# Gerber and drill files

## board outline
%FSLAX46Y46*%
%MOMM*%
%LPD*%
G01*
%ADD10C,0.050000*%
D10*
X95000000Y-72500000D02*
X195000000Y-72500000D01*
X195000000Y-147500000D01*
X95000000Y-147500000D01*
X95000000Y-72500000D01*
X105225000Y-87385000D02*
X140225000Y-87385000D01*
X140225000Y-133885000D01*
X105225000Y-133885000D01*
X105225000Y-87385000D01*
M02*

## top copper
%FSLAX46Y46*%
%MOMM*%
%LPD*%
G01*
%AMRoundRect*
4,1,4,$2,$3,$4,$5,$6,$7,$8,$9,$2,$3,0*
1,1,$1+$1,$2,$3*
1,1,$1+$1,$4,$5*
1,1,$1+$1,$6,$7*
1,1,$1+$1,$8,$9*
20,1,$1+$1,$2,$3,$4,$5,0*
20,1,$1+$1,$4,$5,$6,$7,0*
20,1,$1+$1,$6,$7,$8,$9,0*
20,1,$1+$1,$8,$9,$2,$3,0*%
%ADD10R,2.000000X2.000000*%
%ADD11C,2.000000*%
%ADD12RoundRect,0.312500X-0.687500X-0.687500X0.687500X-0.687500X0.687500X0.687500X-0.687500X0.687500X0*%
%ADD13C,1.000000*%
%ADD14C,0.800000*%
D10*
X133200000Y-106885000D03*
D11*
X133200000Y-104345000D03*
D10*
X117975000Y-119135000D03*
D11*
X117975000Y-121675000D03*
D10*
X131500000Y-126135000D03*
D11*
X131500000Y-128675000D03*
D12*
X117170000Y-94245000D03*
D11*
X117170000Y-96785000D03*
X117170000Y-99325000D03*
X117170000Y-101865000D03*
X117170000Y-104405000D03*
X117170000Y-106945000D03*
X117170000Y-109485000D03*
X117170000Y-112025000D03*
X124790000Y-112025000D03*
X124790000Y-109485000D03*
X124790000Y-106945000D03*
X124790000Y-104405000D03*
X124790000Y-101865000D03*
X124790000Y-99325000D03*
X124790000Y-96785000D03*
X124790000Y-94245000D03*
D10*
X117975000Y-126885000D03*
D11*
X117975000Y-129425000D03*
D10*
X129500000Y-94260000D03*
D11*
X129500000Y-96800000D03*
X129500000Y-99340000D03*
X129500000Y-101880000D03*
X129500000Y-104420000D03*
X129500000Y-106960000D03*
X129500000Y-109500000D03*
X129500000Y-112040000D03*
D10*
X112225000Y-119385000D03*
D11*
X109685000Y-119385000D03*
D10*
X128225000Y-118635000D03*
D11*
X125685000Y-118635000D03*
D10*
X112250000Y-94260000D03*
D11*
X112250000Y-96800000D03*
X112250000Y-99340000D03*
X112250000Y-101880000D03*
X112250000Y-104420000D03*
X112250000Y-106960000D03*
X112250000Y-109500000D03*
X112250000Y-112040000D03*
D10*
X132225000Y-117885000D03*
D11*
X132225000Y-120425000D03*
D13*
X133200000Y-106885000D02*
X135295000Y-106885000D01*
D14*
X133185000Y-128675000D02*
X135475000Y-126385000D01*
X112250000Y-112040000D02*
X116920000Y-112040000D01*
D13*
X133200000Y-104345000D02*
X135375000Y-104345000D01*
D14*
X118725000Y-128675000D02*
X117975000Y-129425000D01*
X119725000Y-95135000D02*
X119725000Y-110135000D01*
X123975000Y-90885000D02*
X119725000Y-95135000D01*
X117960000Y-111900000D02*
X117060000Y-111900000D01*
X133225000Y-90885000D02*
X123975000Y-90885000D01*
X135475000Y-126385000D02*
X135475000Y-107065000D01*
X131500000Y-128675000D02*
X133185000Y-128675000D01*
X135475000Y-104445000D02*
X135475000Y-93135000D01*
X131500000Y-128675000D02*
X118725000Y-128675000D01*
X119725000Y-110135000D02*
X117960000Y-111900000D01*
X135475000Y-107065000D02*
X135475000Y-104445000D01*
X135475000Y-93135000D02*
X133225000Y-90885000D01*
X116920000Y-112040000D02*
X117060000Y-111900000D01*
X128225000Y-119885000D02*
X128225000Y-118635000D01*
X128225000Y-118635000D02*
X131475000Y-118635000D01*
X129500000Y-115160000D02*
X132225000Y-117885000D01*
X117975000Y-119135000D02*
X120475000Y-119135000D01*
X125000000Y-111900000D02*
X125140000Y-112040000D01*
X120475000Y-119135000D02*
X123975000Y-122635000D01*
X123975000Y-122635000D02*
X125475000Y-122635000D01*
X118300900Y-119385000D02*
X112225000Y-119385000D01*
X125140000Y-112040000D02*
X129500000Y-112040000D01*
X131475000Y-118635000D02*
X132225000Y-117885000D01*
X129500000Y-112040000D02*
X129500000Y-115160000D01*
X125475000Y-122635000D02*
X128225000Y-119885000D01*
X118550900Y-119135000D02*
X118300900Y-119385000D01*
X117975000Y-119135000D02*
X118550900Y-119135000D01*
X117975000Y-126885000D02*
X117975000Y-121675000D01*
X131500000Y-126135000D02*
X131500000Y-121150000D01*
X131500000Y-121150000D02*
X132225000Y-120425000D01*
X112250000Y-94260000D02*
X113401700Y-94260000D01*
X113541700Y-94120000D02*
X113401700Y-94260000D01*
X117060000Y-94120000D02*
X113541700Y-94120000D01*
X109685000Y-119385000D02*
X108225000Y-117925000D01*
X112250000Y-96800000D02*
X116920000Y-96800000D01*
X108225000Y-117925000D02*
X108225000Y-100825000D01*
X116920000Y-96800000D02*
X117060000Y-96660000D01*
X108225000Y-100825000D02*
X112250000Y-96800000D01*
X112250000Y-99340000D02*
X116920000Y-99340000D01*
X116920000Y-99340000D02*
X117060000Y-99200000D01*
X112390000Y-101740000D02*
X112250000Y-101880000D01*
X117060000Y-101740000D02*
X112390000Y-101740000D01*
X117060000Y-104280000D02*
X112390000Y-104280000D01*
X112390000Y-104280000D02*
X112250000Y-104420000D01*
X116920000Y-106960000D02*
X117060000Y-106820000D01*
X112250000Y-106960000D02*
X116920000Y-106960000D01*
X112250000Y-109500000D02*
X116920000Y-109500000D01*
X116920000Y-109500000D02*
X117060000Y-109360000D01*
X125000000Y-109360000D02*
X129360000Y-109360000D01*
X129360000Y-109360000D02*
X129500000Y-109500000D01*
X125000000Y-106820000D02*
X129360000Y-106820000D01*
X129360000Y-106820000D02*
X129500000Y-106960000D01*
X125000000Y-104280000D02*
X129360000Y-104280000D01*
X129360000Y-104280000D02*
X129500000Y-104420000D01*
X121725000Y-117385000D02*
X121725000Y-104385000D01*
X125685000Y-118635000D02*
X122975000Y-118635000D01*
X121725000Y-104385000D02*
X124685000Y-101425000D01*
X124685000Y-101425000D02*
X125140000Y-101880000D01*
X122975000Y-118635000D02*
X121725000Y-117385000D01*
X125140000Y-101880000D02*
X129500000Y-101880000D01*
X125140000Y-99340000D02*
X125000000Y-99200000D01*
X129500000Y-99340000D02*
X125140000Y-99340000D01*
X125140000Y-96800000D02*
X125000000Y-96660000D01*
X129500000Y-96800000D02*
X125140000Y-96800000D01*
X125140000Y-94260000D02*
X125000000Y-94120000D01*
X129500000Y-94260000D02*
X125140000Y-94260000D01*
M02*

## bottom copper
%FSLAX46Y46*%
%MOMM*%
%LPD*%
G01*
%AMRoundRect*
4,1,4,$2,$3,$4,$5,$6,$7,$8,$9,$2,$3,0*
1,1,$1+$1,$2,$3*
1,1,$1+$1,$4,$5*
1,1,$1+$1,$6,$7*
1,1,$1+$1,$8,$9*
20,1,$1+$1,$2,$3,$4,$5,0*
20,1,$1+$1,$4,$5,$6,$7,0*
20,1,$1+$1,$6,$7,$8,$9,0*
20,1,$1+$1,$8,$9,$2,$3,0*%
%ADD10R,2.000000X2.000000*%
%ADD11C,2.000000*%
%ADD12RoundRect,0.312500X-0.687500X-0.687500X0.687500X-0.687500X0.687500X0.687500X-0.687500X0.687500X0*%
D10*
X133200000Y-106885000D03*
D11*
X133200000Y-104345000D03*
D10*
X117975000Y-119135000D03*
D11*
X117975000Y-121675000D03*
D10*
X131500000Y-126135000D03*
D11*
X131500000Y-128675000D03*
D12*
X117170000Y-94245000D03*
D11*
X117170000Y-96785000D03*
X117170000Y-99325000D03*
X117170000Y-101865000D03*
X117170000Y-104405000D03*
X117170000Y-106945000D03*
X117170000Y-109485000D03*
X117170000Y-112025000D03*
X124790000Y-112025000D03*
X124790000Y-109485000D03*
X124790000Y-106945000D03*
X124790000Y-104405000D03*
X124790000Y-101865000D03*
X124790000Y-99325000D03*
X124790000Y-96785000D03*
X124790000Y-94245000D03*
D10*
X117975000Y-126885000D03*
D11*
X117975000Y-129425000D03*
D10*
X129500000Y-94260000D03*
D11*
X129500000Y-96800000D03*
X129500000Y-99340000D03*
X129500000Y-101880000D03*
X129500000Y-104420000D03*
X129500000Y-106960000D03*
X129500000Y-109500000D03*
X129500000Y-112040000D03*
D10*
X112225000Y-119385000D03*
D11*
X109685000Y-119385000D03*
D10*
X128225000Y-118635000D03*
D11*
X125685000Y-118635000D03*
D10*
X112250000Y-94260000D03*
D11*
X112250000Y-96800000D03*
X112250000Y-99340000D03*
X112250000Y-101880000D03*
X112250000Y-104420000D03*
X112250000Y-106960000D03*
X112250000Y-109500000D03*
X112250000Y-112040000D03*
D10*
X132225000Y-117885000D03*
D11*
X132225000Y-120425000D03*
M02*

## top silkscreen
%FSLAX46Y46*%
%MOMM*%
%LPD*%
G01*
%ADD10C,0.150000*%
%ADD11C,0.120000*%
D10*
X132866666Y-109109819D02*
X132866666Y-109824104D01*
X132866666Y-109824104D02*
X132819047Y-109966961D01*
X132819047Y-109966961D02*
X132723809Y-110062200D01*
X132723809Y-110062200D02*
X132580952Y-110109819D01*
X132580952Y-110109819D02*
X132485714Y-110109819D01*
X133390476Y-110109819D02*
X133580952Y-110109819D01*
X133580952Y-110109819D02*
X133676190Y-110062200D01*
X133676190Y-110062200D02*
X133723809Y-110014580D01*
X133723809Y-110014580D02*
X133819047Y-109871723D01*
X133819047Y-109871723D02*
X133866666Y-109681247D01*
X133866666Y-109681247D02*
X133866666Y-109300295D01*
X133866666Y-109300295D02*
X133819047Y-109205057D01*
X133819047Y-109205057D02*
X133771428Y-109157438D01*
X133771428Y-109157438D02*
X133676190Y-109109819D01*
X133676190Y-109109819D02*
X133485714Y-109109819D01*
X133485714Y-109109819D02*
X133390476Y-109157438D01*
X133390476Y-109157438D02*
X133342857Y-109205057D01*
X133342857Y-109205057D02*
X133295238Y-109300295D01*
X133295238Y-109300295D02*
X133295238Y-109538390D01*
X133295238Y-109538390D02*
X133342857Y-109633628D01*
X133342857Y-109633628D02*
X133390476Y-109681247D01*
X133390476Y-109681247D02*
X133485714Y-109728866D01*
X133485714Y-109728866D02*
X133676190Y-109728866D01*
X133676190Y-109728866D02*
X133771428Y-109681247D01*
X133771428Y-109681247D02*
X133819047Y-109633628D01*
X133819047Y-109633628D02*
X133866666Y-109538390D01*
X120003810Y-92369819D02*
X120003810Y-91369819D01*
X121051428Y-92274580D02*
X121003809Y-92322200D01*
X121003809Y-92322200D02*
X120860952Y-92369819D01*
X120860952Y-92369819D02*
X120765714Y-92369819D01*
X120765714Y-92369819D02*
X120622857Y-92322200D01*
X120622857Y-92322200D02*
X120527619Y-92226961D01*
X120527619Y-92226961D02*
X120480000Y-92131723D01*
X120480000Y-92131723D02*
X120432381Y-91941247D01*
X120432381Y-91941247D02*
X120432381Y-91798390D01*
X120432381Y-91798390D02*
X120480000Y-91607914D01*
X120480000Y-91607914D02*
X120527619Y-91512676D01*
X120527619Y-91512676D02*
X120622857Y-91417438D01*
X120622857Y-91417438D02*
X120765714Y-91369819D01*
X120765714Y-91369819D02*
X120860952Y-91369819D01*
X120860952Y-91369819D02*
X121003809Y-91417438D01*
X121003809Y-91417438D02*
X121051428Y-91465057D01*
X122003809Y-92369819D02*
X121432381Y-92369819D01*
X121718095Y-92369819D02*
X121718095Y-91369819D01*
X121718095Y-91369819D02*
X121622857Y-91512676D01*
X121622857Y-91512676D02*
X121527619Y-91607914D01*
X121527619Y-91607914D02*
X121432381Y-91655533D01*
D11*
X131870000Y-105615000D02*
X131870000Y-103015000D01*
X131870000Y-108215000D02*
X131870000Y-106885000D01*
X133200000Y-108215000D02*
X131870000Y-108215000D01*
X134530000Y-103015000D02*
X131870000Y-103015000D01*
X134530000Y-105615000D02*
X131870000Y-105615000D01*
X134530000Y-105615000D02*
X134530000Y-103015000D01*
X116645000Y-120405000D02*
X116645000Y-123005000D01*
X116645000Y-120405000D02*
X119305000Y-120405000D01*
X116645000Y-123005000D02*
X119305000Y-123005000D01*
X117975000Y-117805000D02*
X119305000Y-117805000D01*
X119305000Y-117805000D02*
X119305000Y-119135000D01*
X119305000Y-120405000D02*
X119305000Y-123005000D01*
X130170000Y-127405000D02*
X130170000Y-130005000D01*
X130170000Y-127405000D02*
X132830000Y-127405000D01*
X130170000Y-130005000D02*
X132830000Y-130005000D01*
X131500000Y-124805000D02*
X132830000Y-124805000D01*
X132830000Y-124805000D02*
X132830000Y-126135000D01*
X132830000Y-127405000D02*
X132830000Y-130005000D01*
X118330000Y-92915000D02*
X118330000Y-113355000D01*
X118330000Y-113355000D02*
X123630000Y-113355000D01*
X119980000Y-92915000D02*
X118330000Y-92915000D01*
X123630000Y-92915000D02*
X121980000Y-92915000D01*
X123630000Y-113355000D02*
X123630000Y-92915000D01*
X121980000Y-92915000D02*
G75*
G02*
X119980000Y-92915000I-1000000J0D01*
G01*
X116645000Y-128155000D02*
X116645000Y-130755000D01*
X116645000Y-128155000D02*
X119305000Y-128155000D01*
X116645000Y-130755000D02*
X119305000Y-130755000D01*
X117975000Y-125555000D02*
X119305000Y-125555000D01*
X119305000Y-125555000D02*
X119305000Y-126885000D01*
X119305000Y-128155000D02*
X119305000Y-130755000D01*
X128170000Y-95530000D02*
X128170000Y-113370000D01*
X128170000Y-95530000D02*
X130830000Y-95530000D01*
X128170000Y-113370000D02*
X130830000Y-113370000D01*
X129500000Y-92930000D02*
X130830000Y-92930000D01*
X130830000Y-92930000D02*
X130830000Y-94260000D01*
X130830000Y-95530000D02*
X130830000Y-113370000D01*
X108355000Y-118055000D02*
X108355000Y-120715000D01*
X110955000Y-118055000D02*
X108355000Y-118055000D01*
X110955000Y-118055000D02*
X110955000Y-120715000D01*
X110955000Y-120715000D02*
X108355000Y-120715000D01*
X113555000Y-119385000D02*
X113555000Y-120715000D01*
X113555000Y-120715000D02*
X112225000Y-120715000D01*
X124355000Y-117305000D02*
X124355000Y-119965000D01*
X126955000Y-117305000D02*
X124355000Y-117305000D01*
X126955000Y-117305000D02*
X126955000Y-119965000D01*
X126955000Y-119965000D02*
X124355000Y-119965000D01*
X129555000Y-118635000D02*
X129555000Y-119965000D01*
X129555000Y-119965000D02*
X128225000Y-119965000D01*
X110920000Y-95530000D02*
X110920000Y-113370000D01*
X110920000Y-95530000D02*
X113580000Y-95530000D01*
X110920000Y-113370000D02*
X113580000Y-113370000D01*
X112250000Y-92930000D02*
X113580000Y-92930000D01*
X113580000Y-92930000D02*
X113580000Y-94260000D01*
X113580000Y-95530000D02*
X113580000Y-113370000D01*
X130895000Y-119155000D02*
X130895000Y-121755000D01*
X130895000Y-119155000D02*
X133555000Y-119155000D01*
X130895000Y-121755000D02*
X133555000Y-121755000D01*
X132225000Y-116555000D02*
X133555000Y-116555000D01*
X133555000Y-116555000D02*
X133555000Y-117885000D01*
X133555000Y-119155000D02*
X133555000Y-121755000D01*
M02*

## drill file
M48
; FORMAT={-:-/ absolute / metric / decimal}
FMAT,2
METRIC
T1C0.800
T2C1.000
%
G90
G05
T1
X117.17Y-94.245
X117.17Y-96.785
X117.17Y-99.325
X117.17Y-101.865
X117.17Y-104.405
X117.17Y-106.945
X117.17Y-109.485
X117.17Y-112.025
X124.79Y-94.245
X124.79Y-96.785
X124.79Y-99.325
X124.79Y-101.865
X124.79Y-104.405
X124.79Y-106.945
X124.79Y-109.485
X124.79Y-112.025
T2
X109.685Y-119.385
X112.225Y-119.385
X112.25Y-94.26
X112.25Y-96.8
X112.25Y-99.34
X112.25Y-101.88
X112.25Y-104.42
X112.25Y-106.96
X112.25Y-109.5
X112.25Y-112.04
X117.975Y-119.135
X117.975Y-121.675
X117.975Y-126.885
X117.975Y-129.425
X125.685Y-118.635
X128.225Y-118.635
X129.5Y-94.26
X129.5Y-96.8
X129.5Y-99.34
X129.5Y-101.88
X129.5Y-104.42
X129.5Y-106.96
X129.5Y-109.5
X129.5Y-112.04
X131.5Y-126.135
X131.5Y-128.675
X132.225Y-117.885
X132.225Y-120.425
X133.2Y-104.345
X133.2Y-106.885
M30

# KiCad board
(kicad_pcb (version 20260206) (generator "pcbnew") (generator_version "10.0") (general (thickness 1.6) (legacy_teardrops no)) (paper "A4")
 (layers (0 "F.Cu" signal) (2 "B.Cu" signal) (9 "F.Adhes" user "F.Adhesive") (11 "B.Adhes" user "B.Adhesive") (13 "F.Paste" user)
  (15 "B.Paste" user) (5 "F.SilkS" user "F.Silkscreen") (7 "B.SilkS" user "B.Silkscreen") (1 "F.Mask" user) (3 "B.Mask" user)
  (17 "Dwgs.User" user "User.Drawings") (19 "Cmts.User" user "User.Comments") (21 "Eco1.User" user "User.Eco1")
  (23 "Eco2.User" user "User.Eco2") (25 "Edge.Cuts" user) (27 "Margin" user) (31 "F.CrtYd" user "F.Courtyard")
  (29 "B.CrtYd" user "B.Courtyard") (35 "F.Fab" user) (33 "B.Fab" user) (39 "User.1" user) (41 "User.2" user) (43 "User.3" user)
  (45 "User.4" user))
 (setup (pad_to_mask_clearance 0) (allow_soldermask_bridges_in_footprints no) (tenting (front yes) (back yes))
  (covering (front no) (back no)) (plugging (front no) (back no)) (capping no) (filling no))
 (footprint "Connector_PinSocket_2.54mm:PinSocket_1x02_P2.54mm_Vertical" (layer "F.Cu") (at 133.2 106.885 180)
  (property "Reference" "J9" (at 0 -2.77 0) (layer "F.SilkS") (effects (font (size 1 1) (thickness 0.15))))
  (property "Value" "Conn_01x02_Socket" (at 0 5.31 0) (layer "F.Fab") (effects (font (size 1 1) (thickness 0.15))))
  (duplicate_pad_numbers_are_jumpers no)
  (fp_line (start 1.33 1.27) (end 1.33 3.87) (stroke (width 0.12) (type solid)) (layer "F.SilkS"))
  (fp_line (start 1.33 -1.33) (end 1.33 0) (stroke (width 0.12) (type solid)) (layer "F.SilkS"))
  (fp_line (start 0 -1.33) (end 1.33 -1.33) (stroke (width 0.12) (type solid)) (layer "F.SilkS"))
  (fp_line (start -1.33 3.87) (end 1.33 3.87) (stroke (width 0.12) (type solid)) (layer "F.SilkS"))
  (fp_line (start -1.33 1.27) (end 1.33 1.27) (stroke (width 0.12) (type solid)) (layer "F.SilkS"))
  (fp_line (start -1.33 1.27) (end -1.33 3.87) (stroke (width 0.12) (type solid)) (layer "F.SilkS"))
  (pad "1" thru_hole rect (at 0 0 180) (size 2 2) (drill 1) (layers "*.Cu" "*.Mask") (remove_unused_layers no) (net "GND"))
  (pad "2" thru_hole circle (at 0 2.54 180) (size 2 2) (drill 1) (layers "*.Cu" "*.Mask") (remove_unused_layers no) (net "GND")))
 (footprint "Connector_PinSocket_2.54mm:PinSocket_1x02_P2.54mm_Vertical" (layer "F.Cu") (at 117.975 119.135)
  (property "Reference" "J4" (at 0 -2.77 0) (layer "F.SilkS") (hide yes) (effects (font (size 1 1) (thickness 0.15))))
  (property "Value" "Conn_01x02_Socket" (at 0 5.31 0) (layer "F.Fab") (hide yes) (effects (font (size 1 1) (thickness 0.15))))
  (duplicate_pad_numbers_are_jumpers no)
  (fp_line (start -1.33 1.27) (end -1.33 3.87) (stroke (width 0.12) (type solid)) (layer "F.SilkS"))
  (fp_line (start -1.33 1.27) (end 1.33 1.27) (stroke (width 0.12) (type solid)) (layer "F.SilkS"))
  (fp_line (start -1.33 3.87) (end 1.33 3.87) (stroke (width 0.12) (type solid)) (layer "F.SilkS"))
  (fp_line (start 0 -1.33) (end 1.33 -1.33) (stroke (width 0.12) (type solid)) (layer "F.SilkS"))
  (fp_line (start 1.33 -1.33) (end 1.33 0) (stroke (width 0.12) (type solid)) (layer "F.SilkS"))
  (fp_line (start 1.33 1.27) (end 1.33 3.87) (stroke (width 0.12) (type solid)) (layer "F.SilkS"))
  (pad "1" thru_hole rect (at 0 0) (size 2 2) (drill 1) (layers "*.Cu" "*.Mask") (remove_unused_layers no) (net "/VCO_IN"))
  (pad "2" thru_hole circle (at 0 2.54) (size 2 2) (drill 1) (layers "*.Cu" "*.Mask") (remove_unused_layers no) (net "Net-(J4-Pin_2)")))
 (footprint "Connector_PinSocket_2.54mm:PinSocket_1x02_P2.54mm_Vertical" (layer "F.Cu") (at 131.5 126.135)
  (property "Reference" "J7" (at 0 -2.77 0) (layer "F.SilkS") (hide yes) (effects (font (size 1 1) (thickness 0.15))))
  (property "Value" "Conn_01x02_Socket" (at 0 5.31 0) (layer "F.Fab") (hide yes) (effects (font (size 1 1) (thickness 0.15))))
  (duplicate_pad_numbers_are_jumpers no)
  (fp_line (start -1.33 1.27) (end -1.33 3.87) (stroke (width 0.12) (type solid)) (layer "F.SilkS"))
  (fp_line (start -1.33 1.27) (end 1.33 1.27) (stroke (width 0.12) (type solid)) (layer "F.SilkS"))
  (fp_line (start -1.33 3.87) (end 1.33 3.87) (stroke (width 0.12) (type solid)) (layer "F.SilkS"))
  (fp_line (start 0 -1.33) (end 1.33 -1.33) (stroke (width 0.12) (type solid)) (layer "F.SilkS"))
  (fp_line (start 1.33 -1.33) (end 1.33 0) (stroke (width 0.12) (type solid)) (layer "F.SilkS"))
  (fp_line (start 1.33 1.27) (end 1.33 3.87) (stroke (width 0.12) (type solid)) (layer "F.SilkS"))
  (pad "1" thru_hole rect (at 0 0) (size 2 2) (drill 1) (layers "*.Cu" "*.Mask") (remove_unused_layers no) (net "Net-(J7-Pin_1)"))
  (pad "2" thru_hole circle (at 0 2.54) (size 2 2) (drill 1) (layers "*.Cu" "*.Mask") (remove_unused_layers no) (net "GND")))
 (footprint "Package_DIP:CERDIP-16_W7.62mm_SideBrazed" (layer "F.Cu") (at 117.17 94.245)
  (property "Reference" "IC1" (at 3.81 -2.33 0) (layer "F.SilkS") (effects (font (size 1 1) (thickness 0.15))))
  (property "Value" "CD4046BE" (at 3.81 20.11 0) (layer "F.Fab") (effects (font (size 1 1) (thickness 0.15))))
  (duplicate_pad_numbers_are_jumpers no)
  (fp_line (start 1.16 -1.33) (end 1.16 19.11) (stroke (width 0.12) (type solid)) (layer "F.SilkS"))
  (fp_line (start 1.16 19.11) (end 6.46 19.11) (stroke (width 0.12) (type solid)) (layer "F.SilkS"))
  (fp_line (start 2.81 -1.33) (end 1.16 -1.33) (stroke (width 0.12) (type solid)) (layer "F.SilkS"))
  (fp_line (start 6.46 -1.33) (end 4.81 -1.33) (stroke (width 0.12) (type solid)) (layer "F.SilkS"))
  (fp_line (start 6.46 19.11) (end 6.46 -1.33) (stroke (width 0.12) (type solid)) (layer "F.SilkS"))
  (fp_arc (start 4.81 -1.33) (mid 3.81 -0.33) (end 2.81 -1.33) (stroke (width 0.12) (type solid)) (layer "F.SilkS"))
  (pad "1" thru_hole roundrect (at 0 0) (size 2 2) (drill 0.8) (layers "*.Cu" "*.Mask") (remove_unused_layers no) (roundrect_rratio 0.15625)
   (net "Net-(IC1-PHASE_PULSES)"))
  (pad "2" thru_hole circle (at 0 2.54) (size 2 2) (drill 0.8) (layers "*.Cu" "*.Mask") (remove_unused_layers no) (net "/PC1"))
  (pad "3" thru_hole circle (at 0 5.08) (size 2 2) (drill 0.8) (layers "*.Cu" "*.Mask") (remove_unused_layers no)
   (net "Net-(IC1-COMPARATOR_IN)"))
  (pad "4" thru_hole circle (at 0 7.62) (size 2 2) (drill 0.8) (layers "*.Cu" "*.Mask") (remove_unused_layers no) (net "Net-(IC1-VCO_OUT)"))
  (pad "5" thru_hole circle (at 0 10.16) (size 2 2) (drill 0.8) (layers "*.Cu" "*.Mask") (remove_unused_layers no) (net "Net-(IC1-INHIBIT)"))
  (pad "6" thru_hole circle (at 0 12.7) (size 2 2) (drill 0.8) (layers "*.Cu" "*.Mask") (remove_unused_layers no) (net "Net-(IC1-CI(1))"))
  (pad "7" thru_hole circle (at 0 15.24) (size 2 2) (drill 0.8) (layers "*.Cu" "*.Mask") (remove_unused_layers no) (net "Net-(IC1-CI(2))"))
  (pad "8" thru_hole circle (at 0 17.78) (size 2 2) (drill 0.8) (layers "*.Cu" "*.Mask") (remove_unused_layers no) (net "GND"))
  (pad "9" thru_hole circle (at 7.62 17.78) (size 2 2) (drill 0.8) (layers "*.Cu" "*.Mask") (remove_unused_layers no) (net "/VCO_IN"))
  (pad "10" thru_hole circle (at 7.62 15.24) (size 2 2) (drill 0.8) (layers "*.Cu" "*.Mask") (remove_unused_layers no)
   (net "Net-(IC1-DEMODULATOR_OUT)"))
  (pad "11" thru_hole circle (at 7.62 12.7) (size 2 2) (drill 0.8) (layers "*.Cu" "*.Mask") (remove_unused_layers no)
   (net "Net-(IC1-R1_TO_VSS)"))
  (pad "12" thru_hole circle (at 7.62 10.16) (size 2 2) (drill 0.8) (layers "*.Cu" "*.Mask") (remove_unused_layers no)
   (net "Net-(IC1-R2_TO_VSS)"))
  (pad "13" thru_hole circle (at 7.62 7.62) (size 2 2) (drill 0.8) (layers "*.Cu" "*.Mask") (remove_unused_layers no) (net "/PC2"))
  (pad "14" thru_hole circle (at 7.62 5.08) (size 2 2) (drill 0.8) (layers "*.Cu" "*.Mask") (remove_unused_layers no)
   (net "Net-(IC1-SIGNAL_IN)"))
  (pad "15" thru_hole circle (at 7.62 2.54) (size 2 2) (drill 0.8) (layers "*.Cu" "*.Mask") (remove_unused_layers no)
   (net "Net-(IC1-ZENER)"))
  (pad "16" thru_hole circle (at 7.62 0) (size 2 2) (drill 0.8) (layers "*.Cu" "*.Mask") (remove_unused_layers no) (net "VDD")))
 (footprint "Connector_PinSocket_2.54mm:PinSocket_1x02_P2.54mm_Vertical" (layer "F.Cu") (at 117.975 126.885)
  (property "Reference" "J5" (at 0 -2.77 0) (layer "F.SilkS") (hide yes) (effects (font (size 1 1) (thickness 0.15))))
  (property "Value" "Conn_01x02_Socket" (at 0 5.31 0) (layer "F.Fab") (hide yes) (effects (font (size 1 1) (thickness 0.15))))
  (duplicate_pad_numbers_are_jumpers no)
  (fp_line (start -1.33 1.27) (end -1.33 3.87) (stroke (width 0.12) (type solid)) (layer "F.SilkS"))
  (fp_line (start -1.33 1.27) (end 1.33 1.27) (stroke (width 0.12) (type solid)) (layer "F.SilkS"))
  (fp_line (start -1.33 3.87) (end 1.33 3.87) (stroke (width 0.12) (type solid)) (layer "F.SilkS"))
  (fp_line (start 0 -1.33) (end 1.33 -1.33) (stroke (width 0.12) (type solid)) (layer "F.SilkS"))
  (fp_line (start 1.33 -1.33) (end 1.33 0) (stroke (width 0.12) (type solid)) (layer "F.SilkS"))
  (fp_line (start 1.33 1.27) (end 1.33 3.87) (stroke (width 0.12) (type solid)) (layer "F.SilkS"))
  (pad "1" thru_hole rect (at 0 0) (size 2 2) (drill 1) (layers "*.Cu" "*.Mask") (remove_unused_layers no) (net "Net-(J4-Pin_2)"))
  (pad "2" thru_hole circle (at 0 2.54) (size 2 2) (drill 1) (layers "*.Cu" "*.Mask") (remove_unused_layers no) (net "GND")))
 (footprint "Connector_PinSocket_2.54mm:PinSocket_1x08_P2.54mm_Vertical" (layer "F.Cu") (at 129.5 94.26)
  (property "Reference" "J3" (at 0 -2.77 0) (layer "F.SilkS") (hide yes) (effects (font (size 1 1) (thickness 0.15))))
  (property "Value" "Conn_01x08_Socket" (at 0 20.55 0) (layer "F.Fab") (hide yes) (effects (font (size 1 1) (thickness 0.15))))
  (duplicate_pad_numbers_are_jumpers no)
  (fp_line (start -1.33 1.27) (end -1.33 19.11) (stroke (width 0.12) (type solid)) (layer "F.SilkS"))
  (fp_line (start -1.33 1.27) (end 1.33 1.27) (stroke (width 0.12) (type solid)) (layer "F.SilkS"))
  (fp_line (start -1.33 19.11) (end 1.33 19.11) (stroke (width 0.12) (type solid)) (layer "F.SilkS"))
  (fp_line (start 0 -1.33) (end 1.33 -1.33) (stroke (width 0.12) (type solid)) (layer "F.SilkS"))
  (fp_line (start 1.33 -1.33) (end 1.33 0) (stroke (width 0.12) (type solid)) (layer "F.SilkS"))
  (fp_line (start 1.33 1.27) (end 1.33 19.11) (stroke (width 0.12) (type solid)) (layer "F.SilkS"))
  (pad "1" thru_hole rect (at 0 0) (size 2 2) (drill 1) (layers "*.Cu" "*.Mask") (remove_unused_layers no) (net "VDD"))
  (pad "2" thru_hole circle (at 0 2.54) (size 2 2) (drill 1) (layers "*.Cu" "*.Mask") (remove_unused_layers no) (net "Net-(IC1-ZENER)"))
  (pad "3" thru_hole circle (at 0 5.08) (size 2 2) (drill 1) (layers "*.Cu" "*.Mask") (remove_unused_layers no) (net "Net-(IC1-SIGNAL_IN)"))
  (pad "4" thru_hole circle (at 0 7.62) (size 2 2) (drill 1) (layers "*.Cu" "*.Mask") (remove_unused_layers no) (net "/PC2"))
  (pad "5" thru_hole circle (at 0 10.16) (size 2 2) (drill 1) (layers "*.Cu" "*.Mask") (remove_unused_layers no) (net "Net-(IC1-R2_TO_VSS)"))
  (pad "6" thru_hole circle (at 0 12.7) (size 2 2) (drill 1) (layers "*.Cu" "*.Mask") (remove_unused_layers no) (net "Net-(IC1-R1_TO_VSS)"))
  (pad "7" thru_hole circle (at 0 15.24) (size 2 2) (drill 1) (layers "*.Cu" "*.Mask") (remove_unused_layers no)
   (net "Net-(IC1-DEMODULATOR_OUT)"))
  (pad "8" thru_hole circle (at 0 17.78) (size 2 2) (drill 1) (layers "*.Cu" "*.Mask") (remove_unused_layers no) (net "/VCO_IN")))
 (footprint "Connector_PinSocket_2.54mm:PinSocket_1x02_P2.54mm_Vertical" (layer "F.Cu") (at 112.225 119.385 -90)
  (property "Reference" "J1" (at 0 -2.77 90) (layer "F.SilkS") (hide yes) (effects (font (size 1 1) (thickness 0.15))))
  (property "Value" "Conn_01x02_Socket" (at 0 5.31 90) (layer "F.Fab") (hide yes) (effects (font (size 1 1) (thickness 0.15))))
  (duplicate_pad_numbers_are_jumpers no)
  (fp_line (start -1.33 3.87) (end 1.33 3.87) (stroke (width 0.12) (type solid)) (layer "F.SilkS"))
  (fp_line (start -1.33 1.27) (end -1.33 3.87) (stroke (width 0.12) (type solid)) (layer "F.SilkS"))
  (fp_line (start -1.33 1.27) (end 1.33 1.27) (stroke (width 0.12) (type solid)) (layer "F.SilkS"))
  (fp_line (start 1.33 1.27) (end 1.33 3.87) (stroke (width 0.12) (type solid)) (layer "F.SilkS"))
  (fp_line (start 0 -1.33) (end 1.33 -1.33) (stroke (width 0.12) (type solid)) (layer "F.SilkS"))
  (fp_line (start 1.33 -1.33) (end 1.33 0) (stroke (width 0.12) (type solid)) (layer "F.SilkS"))
  (pad "1" thru_hole rect (at 0 0 270) (size 2 2) (drill 1) (layers "*.Cu" "*.Mask") (remove_unused_layers no) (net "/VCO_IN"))
  (pad "2" thru_hole circle (at 0 2.54 270) (size 2 2) (drill 1) (layers "*.Cu" "*.Mask") (remove_unused_layers no) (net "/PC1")))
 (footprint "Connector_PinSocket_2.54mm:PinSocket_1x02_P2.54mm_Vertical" (layer "F.Cu") (at 128.225 118.635 -90)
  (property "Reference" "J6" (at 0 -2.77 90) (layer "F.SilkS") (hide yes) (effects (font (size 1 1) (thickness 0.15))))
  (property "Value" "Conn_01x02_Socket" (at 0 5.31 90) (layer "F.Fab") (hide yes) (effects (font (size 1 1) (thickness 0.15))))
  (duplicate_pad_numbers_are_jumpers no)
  (fp_line (start -1.33 3.87) (end 1.33 3.87) (stroke (width 0.12) (type solid)) (layer "F.SilkS"))
  (fp_line (start -1.33 1.27) (end -1.33 3.87) (stroke (width 0.12) (type solid)) (layer "F.SilkS"))
  (fp_line (start -1.33 1.27) (end 1.33 1.27) (stroke (width 0.12) (type solid)) (layer "F.SilkS"))
  (fp_line (start 1.33 1.27) (end 1.33 3.87) (stroke (width 0.12) (type solid)) (layer "F.SilkS"))
  (fp_line (start 0 -1.33) (end 1.33 -1.33) (stroke (width 0.12) (type solid)) (layer "F.SilkS"))
  (fp_line (start 1.33 -1.33) (end 1.33 0) (stroke (width 0.12) (type solid)) (layer "F.SilkS"))
  (pad "1" thru_hole rect (at 0 0 270) (size 2 2) (drill 1) (layers "*.Cu" "*.Mask") (remove_unused_layers no) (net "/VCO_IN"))
  (pad "2" thru_hole circle (at 0 2.54 270) (size 2 2) (drill 1) (layers "*.Cu" "*.Mask") (remove_unused_layers no) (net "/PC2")))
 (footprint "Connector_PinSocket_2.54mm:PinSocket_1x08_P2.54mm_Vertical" (layer "F.Cu") (at 112.25 94.26)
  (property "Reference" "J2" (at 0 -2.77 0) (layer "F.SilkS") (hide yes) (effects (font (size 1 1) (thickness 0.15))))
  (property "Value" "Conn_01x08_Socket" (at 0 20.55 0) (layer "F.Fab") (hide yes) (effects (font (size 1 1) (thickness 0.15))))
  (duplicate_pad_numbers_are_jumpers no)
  (fp_line (start -1.33 1.27) (end -1.33 19.11) (stroke (width 0.12) (type solid)) (layer "F.SilkS"))
  (fp_line (start -1.33 1.27) (end 1.33 1.27) (stroke (width 0.12) (type solid)) (layer "F.SilkS"))
  (fp_line (start -1.33 19.11) (end 1.33 19.11) (stroke (width 0.12) (type solid)) (layer "F.SilkS"))
  (fp_line (start 0 -1.33) (end 1.33 -1.33) (stroke (width 0.12) (type solid)) (layer "F.SilkS"))
  (fp_line (start 1.33 -1.33) (end 1.33 0) (stroke (width 0.12) (type solid)) (layer "F.SilkS"))
  (fp_line (start 1.33 1.27) (end 1.33 19.11) (stroke (width 0.12) (type solid)) (layer "F.SilkS"))
  (pad "1" thru_hole rect (at 0 0) (size 2 2) (drill 1) (layers "*.Cu" "*.Mask") (remove_unused_layers no) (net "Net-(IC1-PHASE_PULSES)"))
  (pad "2" thru_hole circle (at 0 2.54) (size 2 2) (drill 1) (layers "*.Cu" "*.Mask") (remove_unused_layers no) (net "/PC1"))
  (pad "3" thru_hole circle (at 0 5.08) (size 2 2) (drill 1) (layers "*.Cu" "*.Mask") (remove_unused_layers no)
   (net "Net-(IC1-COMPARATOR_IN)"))
  (pad "4" thru_hole circle (at 0 7.62) (size 2 2) (drill 1) (layers "*.Cu" "*.Mask") (remove_unused_layers no) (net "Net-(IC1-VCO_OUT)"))
  (pad "5" thru_hole circle (at 0 10.16) (size 2 2) (drill 1) (layers "*.Cu" "*.Mask") (remove_unused_layers no) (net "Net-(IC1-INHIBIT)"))
  (pad "6" thru_hole circle (at 0 12.7) (size 2 2) (drill 1) (layers "*.Cu" "*.Mask") (remove_unused_layers no) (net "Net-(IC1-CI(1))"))
  (pad "7" thru_hole circle (at 0 15.24) (size 2 2) (drill 1) (layers "*.Cu" "*.Mask") (remove_unused_layers no) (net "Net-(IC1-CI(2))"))
  (pad "8" thru_hole circle (at 0 17.78) (size 2 2) (drill 1) (layers "*.Cu" "*.Mask") (remove_unused_layers no) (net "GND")))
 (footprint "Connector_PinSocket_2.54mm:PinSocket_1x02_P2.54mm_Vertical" (layer "F.Cu") (at 132.225 117.885)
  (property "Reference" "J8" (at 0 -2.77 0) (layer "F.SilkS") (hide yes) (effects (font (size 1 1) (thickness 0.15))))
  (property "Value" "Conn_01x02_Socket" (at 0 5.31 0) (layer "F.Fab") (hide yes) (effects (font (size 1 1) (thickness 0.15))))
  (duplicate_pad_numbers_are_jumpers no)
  (fp_line (start -1.33 1.27) (end -1.33 3.87) (stroke (width 0.12) (type solid)) (layer "F.SilkS"))
  (fp_line (start -1.33 1.27) (end 1.33 1.27) (stroke (width 0.12) (type solid)) (layer "F.SilkS"))
  (fp_line (start -1.33 3.87) (end 1.33 3.87) (stroke (width 0.12) (type solid)) (layer "F.SilkS"))
  (fp_line (start 0 -1.33) (end 1.33 -1.33) (stroke (width 0.12) (type solid)) (layer "F.SilkS"))
  (fp_line (start 1.33 -1.33) (end 1.33 0) (stroke (width 0.12) (type solid)) (layer "F.SilkS"))
  (fp_line (start 1.33 1.27) (end 1.33 3.87) (stroke (width 0.12) (type solid)) (layer "F.SilkS"))
  (pad "1" thru_hole rect (at 0 0) (size 2 2) (drill 1) (layers "*.Cu" "*.Mask") (remove_unused_layers no) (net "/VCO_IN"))
  (pad "2" thru_hole circle (at 0 2.54) (size 2 2) (drill 1) (layers "*.Cu" "*.Mask") (remove_unused_layers no) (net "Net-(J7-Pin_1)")))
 (gr_rect (start 95 72.5) (end 195 147.5) (stroke (width 0.05) (type default)) (fill no) (layer "Edge.Cuts"))
 (gr_rect (start 105.225 87.385) (end 140.225 133.885) (stroke (width 0.05) (type default)) (fill no) (layer "Edge.Cuts"))
 (segment (start 133.2 106.885) (end 135.295 106.885) (width 1) (layer "F.Cu") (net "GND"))
 (segment (start 133.185 128.675) (end 135.475 126.385) (width 0.8) (layer "F.Cu") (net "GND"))
 (segment (start 112.25 112.04) (end 116.92 112.04) (width 0.8) (layer "F.Cu") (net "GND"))
 (segment (start 133.2 104.345) (end 135.375 104.345) (width 1) (layer "F.Cu") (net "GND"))
 (segment (start 118.725 128.675) (end 117.975 129.425) (width 0.8) (layer "F.Cu") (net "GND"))
 (segment (start 119.725 95.135) (end 119.725 110.135) (width 0.8) (layer "F.Cu") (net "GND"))
 (segment (start 123.975 90.885) (end 119.725 95.135) (width 0.8) (layer "F.Cu") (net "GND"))
 (segment (start 117.96 111.9) (end 117.06 111.9) (width 0.8) (layer "F.Cu") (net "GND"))
 (segment (start 133.225 90.885) (end 123.975 90.885) (width 0.8) (layer "F.Cu") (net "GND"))
 (segment (start 135.475 126.385) (end 135.475 107.065) (width 0.8) (layer "F.Cu") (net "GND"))
 (segment (start 131.5 128.675) (end 133.185 128.675) (width 0.8) (layer "F.Cu") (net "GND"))
 (segment (start 135.475 104.445) (end 135.475 93.135) (width 0.8) (layer "F.Cu") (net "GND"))
 (segment (start 131.5 128.675) (end 118.725 128.675) (width 0.8) (layer "F.Cu") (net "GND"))
 (segment (start 119.725 110.135) (end 117.96 111.9) (width 0.8) (layer "F.Cu") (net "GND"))
 (segment (start 135.475 107.065) (end 135.475 104.445) (width 0.8) (layer "F.Cu") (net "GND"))
 (segment (start 135.475 93.135) (end 133.225 90.885) (width 0.8) (layer "F.Cu") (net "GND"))
 (segment (start 116.92 112.04) (end 117.06 111.9) (width 0.8) (layer "F.Cu") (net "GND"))
 (segment (start 128.225 119.885) (end 128.225 118.635) (width 0.8) (layer "F.Cu") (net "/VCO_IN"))
 (segment (start 128.225 118.635) (end 131.475 118.635) (width 0.8) (layer "F.Cu") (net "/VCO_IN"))
 (segment (start 129.5 115.16) (end 132.225 117.885) (width 0.8) (layer "F.Cu") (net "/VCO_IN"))
 (segment (start 117.975 119.135) (end 120.475 119.135) (width 0.8) (layer "F.Cu") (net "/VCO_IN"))
 (segment (start 125 111.9) (end 125.14 112.04) (width 0.8) (layer "F.Cu") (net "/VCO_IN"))
 (segment (start 120.475 119.135) (end 123.975 122.635) (width 0.8) (layer "F.Cu") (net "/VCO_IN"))
 (segment (start 123.975 122.635) (end 125.475 122.635) (width 0.8) (layer "F.Cu") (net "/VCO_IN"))
 (segment (start 118.3009 119.385) (end 112.225 119.385) (width 0.8) (layer "F.Cu") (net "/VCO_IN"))
 (segment (start 125.14 112.04) (end 129.5 112.04) (width 0.8) (layer "F.Cu") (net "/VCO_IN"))
 (segment (start 131.475 118.635) (end 132.225 117.885) (width 0.8) (layer "F.Cu") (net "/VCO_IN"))
 (segment (start 129.5 112.04) (end 129.5 115.16) (width 0.8) (layer "F.Cu") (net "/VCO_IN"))
 (segment (start 125.475 122.635) (end 128.225 119.885) (width 0.8) (layer "F.Cu") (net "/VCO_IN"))
 (segment (start 118.5509 119.135) (end 118.3009 119.385) (width 0.8) (layer "F.Cu") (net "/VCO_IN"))
 (segment (start 117.975 119.135) (end 118.5509 119.135) (width 0.8) (layer "F.Cu") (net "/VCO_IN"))
 (segment (start 117.975 126.885) (end 117.975 121.675) (width 0.8) (layer "F.Cu") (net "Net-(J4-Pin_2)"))
 (segment (start 131.5 126.135) (end 131.5 121.15) (width 0.8) (layer "F.Cu") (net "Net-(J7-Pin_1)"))
 (segment (start 131.5 121.15) (end 132.225 120.425) (width 0.8) (layer "F.Cu") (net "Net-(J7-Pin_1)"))
 (segment (start 112.25 94.26) (end 113.4017 94.26) (width 0.8) (layer "F.Cu") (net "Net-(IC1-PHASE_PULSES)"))
 (segment (start 113.5417 94.12) (end 113.4017 94.26) (width 0.8) (layer "F.Cu") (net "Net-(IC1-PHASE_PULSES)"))
 (segment (start 117.06 94.12) (end 113.5417 94.12) (width 0.8) (layer "F.Cu") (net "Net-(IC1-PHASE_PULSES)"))
 (segment (start 109.685 119.385) (end 108.225 117.925) (width 0.8) (layer "F.Cu") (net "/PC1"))
 (segment (start 112.25 96.8) (end 116.92 96.8) (width 0.8) (layer "F.Cu") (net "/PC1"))
 (segment (start 108.225 117.925) (end 108.225 100.825) (width 0.8) (layer "F.Cu") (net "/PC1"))
 (segment (start 116.92 96.8) (end 117.06 96.66) (width 0.8) (layer "F.Cu") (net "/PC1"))
 (segment (start 108.225 100.825) (end 112.25 96.8) (width 0.8) (layer "F.Cu") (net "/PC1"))
 (segment (start 112.25 99.34) (end 116.92 99.34) (width 0.8) (layer "F.Cu") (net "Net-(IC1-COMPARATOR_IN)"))
 (segment (start 116.92 99.34) (end 117.06 99.2) (width 0.8) (layer "F.Cu") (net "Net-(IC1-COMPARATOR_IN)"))
 (segment (start 112.39 101.74) (end 112.25 101.88) (width 0.8) (layer "F.Cu") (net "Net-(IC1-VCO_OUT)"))
 (segment (start 117.06 101.74) (end 112.39 101.74) (width 0.8) (layer "F.Cu") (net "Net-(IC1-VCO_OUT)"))
 (segment (start 117.06 104.28) (end 112.39 104.28) (width 0.8) (layer "F.Cu") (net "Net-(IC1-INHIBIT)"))
 (segment (start 112.39 104.28) (end 112.25 104.42) (width 0.8) (layer "F.Cu") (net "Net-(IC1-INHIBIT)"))
 (segment (start 116.92 106.96) (end 117.06 106.82) (width 0.8) (layer "F.Cu") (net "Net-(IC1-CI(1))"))
 (segment (start 112.25 106.96) (end 116.92 106.96) (width 0.8) (layer "F.Cu") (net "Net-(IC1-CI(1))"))
 (segment (start 112.25 109.5) (end 116.92 109.5) (width 0.8) (layer "F.Cu") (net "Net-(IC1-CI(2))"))
 (segment (start 116.92 109.5) (end 117.06 109.36) (width 0.8) (layer "F.Cu") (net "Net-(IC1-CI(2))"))
 (segment (start 125 109.36) (end 129.36 109.36) (width 0.8) (layer "F.Cu") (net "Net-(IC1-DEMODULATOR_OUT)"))
 (segment (start 129.36 109.36) (end 129.5 109.5) (width 0.8) (layer "F.Cu") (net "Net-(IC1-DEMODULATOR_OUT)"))
 (segment (start 125 106.82) (end 129.36 106.82) (width 0.8) (layer "F.Cu") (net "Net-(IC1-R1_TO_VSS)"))
 (segment (start 129.36 106.82) (end 129.5 106.96) (width 0.8) (layer "F.Cu") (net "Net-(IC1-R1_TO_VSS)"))
 (segment (start 125 104.28) (end 129.36 104.28) (width 0.8) (layer "F.Cu") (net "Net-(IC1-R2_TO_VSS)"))
 (segment (start 129.36 104.28) (end 129.5 104.42) (width 0.8) (layer "F.Cu") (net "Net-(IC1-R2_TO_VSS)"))
 (segment (start 121.725 117.385) (end 121.725 104.385) (width 0.8) (layer "F.Cu") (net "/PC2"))
 (segment (start 125.685 118.635) (end 122.975 118.635) (width 0.8) (layer "F.Cu") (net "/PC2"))
 (segment (start 121.725 104.385) (end 124.685 101.425) (width 0.8) (layer "F.Cu") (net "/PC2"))
 (segment (start 124.685 101.425) (end 125.14 101.88) (width 0.8) (layer "F.Cu") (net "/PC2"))
 (segment (start 122.975 118.635) (end 121.725 117.385) (width 0.8) (layer "F.Cu") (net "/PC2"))
 (segment (start 125.14 101.88) (end 129.5 101.88) (width 0.8) (layer "F.Cu") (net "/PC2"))
 (segment (start 125.14 99.34) (end 125 99.2) (width 0.8) (layer "F.Cu") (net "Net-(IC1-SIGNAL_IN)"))
 (segment (start 129.5 99.34) (end 125.14 99.34) (width 0.8) (layer "F.Cu") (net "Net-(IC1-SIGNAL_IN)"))
 (segment (start 125.14 96.8) (end 125 96.66) (width 0.8) (layer "F.Cu") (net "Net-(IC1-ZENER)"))
 (segment (start 129.5 96.8) (end 125.14 96.8) (width 0.8) (layer "F.Cu") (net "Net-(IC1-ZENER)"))
 (segment (start 125.14 94.26) (end 125 94.12) (width 0.8) (layer "F.Cu") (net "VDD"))
 (segment (start 129.5 94.26) (end 125.14 94.26) (width 0.8) (layer "F.Cu") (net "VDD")))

